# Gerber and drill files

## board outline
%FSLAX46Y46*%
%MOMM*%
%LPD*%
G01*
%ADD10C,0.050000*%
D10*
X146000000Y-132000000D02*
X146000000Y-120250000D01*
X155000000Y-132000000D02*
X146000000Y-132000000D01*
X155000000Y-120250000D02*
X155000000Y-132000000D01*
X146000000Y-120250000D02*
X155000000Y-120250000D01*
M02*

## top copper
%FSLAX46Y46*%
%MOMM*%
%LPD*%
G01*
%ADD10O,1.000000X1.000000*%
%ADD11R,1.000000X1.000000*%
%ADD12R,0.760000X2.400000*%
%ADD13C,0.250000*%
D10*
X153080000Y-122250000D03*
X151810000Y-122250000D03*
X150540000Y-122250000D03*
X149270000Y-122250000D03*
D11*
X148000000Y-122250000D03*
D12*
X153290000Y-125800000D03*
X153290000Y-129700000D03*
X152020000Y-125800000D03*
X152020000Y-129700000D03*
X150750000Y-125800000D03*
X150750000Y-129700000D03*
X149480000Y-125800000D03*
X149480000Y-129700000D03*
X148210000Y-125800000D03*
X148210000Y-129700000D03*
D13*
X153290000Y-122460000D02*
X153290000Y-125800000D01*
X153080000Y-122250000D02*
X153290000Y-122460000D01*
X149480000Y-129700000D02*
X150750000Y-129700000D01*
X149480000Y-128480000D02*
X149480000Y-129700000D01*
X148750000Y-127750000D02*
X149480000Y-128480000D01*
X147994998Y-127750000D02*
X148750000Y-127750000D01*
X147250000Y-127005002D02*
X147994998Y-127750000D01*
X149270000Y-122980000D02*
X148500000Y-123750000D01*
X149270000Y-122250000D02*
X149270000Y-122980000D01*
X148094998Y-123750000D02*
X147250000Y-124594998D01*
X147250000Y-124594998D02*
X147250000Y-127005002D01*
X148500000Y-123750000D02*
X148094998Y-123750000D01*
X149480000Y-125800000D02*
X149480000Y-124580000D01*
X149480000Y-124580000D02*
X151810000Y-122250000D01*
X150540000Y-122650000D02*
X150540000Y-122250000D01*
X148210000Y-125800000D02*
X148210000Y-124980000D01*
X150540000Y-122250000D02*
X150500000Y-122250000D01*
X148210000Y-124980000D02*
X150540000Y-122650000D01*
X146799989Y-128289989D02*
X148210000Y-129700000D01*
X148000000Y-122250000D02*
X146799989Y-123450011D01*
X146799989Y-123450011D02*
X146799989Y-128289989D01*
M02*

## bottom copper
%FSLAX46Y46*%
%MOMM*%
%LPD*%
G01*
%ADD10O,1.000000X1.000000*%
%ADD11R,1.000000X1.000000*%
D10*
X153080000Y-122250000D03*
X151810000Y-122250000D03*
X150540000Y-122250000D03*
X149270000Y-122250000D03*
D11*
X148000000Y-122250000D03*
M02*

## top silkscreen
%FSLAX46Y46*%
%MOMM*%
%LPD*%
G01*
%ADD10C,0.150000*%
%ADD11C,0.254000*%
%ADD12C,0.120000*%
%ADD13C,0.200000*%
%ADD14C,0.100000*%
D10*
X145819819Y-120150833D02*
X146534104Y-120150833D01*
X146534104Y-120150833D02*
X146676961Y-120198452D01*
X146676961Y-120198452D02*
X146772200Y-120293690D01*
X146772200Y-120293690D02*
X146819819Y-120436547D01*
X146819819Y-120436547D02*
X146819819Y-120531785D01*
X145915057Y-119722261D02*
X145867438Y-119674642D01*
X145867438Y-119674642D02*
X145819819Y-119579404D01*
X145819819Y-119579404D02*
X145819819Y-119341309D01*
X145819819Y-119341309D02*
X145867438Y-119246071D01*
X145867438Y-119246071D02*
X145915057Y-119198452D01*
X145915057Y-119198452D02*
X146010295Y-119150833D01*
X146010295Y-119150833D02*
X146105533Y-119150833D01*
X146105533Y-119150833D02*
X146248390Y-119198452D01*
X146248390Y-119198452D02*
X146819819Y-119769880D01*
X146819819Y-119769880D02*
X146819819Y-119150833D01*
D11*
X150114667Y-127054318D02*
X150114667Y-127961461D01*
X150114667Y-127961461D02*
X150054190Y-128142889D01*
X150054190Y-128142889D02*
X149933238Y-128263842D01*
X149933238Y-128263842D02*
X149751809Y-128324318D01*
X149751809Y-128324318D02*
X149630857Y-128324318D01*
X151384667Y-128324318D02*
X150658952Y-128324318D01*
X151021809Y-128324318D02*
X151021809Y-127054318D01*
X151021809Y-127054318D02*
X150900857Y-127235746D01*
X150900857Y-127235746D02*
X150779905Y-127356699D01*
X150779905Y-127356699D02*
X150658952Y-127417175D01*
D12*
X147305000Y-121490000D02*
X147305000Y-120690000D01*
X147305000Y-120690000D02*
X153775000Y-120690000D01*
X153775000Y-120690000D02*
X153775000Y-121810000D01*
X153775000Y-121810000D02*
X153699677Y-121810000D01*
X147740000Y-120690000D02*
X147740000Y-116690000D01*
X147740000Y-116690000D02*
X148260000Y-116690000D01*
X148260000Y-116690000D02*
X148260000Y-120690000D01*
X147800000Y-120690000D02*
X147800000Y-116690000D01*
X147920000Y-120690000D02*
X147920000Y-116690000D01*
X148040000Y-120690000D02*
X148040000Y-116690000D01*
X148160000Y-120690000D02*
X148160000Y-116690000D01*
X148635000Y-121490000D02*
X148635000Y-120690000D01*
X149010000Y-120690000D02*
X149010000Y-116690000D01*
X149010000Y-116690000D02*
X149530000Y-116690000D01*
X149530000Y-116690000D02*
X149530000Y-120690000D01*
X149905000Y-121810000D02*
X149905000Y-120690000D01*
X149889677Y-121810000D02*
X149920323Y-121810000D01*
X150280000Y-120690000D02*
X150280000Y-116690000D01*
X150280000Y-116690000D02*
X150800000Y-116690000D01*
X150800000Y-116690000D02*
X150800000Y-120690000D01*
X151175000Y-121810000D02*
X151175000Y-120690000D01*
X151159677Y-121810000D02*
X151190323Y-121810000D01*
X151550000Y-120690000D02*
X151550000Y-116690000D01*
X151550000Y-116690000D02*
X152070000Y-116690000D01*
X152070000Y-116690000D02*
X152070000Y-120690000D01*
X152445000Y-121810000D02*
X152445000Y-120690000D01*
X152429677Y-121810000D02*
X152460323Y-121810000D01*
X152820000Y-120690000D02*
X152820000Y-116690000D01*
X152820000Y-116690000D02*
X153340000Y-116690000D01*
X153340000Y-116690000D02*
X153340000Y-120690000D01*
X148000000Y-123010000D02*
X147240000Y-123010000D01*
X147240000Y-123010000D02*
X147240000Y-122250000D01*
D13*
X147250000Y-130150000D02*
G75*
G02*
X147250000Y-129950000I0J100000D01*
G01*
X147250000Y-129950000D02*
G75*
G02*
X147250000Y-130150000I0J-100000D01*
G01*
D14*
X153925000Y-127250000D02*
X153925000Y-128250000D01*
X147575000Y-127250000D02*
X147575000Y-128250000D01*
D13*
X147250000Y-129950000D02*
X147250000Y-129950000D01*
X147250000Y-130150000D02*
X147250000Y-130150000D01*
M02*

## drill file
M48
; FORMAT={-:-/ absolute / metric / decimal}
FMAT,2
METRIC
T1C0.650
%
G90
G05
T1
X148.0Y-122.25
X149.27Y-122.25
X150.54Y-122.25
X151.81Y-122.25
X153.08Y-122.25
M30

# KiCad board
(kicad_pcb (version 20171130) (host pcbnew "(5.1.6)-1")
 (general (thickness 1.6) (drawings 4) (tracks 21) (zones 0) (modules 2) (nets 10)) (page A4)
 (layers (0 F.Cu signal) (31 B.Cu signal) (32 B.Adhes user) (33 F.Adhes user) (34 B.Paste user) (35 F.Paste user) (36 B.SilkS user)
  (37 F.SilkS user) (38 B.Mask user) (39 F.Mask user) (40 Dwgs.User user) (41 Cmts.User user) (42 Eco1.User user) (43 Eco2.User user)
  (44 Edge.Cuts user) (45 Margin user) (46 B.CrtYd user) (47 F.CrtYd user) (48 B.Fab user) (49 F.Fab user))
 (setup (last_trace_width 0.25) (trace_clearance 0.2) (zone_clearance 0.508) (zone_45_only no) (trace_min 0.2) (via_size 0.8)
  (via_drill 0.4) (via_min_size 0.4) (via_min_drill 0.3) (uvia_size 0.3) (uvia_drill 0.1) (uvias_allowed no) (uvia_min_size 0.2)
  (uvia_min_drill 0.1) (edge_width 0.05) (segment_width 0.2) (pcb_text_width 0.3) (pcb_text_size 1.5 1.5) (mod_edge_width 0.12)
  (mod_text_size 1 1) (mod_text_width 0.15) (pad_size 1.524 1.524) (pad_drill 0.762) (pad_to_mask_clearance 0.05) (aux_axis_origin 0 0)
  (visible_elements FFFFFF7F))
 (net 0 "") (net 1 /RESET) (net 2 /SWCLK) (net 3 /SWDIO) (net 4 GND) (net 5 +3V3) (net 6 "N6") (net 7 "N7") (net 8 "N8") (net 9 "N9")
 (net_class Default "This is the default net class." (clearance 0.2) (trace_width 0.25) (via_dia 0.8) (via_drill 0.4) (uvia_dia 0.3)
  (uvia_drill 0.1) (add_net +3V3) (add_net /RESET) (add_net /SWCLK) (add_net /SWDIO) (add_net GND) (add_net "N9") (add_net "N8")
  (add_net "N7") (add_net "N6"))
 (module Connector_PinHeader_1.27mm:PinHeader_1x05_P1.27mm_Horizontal (layer F.Cu) (at 148 122.25 90)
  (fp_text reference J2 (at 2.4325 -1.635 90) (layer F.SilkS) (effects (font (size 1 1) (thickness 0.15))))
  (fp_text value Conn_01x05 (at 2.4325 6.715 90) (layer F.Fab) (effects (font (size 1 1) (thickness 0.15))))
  (fp_line (start 0.76 -0.695) (end 1.56 -0.695) (layer F.SilkS) (width 0.12))
  (fp_line (start 1.56 -0.695) (end 1.56 5.775) (layer F.SilkS) (width 0.12))
  (fp_line (start 1.56 5.775) (end 0.44 5.775) (layer F.SilkS) (width 0.12))
  (fp_line (start 0.44 5.775) (end 0.44 5.699677) (layer F.SilkS) (width 0.12))
  (fp_line (start 1.56 -0.26) (end 5.56 -0.26) (layer F.SilkS) (width 0.12))
  (fp_line (start 5.56 -0.26) (end 5.56 0.26) (layer F.SilkS) (width 0.12))
  (fp_line (start 5.56 0.26) (end 1.56 0.26) (layer F.SilkS) (width 0.12))
  (fp_line (start 1.56 -0.2) (end 5.56 -0.2) (layer F.SilkS) (width 0.12))
  (fp_line (start 1.56 -0.08) (end 5.56 -0.08) (layer F.SilkS) (width 0.12))
  (fp_line (start 1.56 0.04) (end 5.56 0.04) (layer F.SilkS) (width 0.12))
  (fp_line (start 1.56 0.16) (end 5.56 0.16) (layer F.SilkS) (width 0.12))
  (fp_line (start 0.76 0.635) (end 1.56 0.635) (layer F.SilkS) (width 0.12))
  (fp_line (start 1.56 1.01) (end 5.56 1.01) (layer F.SilkS) (width 0.12))
  (fp_line (start 5.56 1.01) (end 5.56 1.53) (layer F.SilkS) (width 0.12))
  (fp_line (start 5.56 1.53) (end 1.56 1.53) (layer F.SilkS) (width 0.12))
  (fp_line (start 0.44 1.905) (end 1.56 1.905) (layer F.SilkS) (width 0.12))
  (fp_line (start 0.44 1.889677) (end 0.44 1.920323) (layer F.SilkS) (width 0.12))
  (fp_line (start 1.56 2.28) (end 5.56 2.28) (layer F.SilkS) (width 0.12))
  (fp_line (start 5.56 2.28) (end 5.56 2.8) (layer F.SilkS) (width 0.12))
  (fp_line (start 5.56 2.8) (end 1.56 2.8) (layer F.SilkS) (width 0.12))
  (fp_line (start 0.44 3.175) (end 1.56 3.175) (layer F.SilkS) (width 0.12))
  (fp_line (start 0.44 3.159677) (end 0.44 3.190323) (layer F.SilkS) (width 0.12))
  (fp_line (start 1.56 3.55) (end 5.56 3.55) (layer F.SilkS) (width 0.12))
  (fp_line (start 5.56 3.55) (end 5.56 4.07) (layer F.SilkS) (width 0.12))
  (fp_line (start 5.56 4.07) (end 1.56 4.07) (layer F.SilkS) (width 0.12))
  (fp_line (start 0.44 4.445) (end 1.56 4.445) (layer F.SilkS) (width 0.12))
  (fp_line (start 0.44 4.429677) (end 0.44 4.460323) (layer F.SilkS) (width 0.12))
  (fp_line (start 1.56 4.82) (end 5.56 4.82) (layer F.SilkS) (width 0.12))
  (fp_line (start 5.56 4.82) (end 5.56 5.34) (layer F.SilkS) (width 0.12))
  (fp_line (start 5.56 5.34) (end 1.56 5.34) (layer F.SilkS) (width 0.12))
  (fp_line (start -0.76 0) (end -0.76 -0.76) (layer F.SilkS) (width 0.12))
  (fp_line (start -0.76 -0.76) (end 0 -0.76) (layer F.SilkS) (width 0.12))
  (pad 5 thru_hole oval (at 0 5.08 90) (size 1 1) (drill 0.65) (layers *.Cu *.Mask) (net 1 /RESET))
  (pad 4 thru_hole oval (at 0 3.81 90) (size 1 1) (drill 0.65) (layers *.Cu *.Mask) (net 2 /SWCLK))
  (pad 3 thru_hole oval (at 0 2.54 90) (size 1 1) (drill 0.65) (layers *.Cu *.Mask) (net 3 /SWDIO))
  (pad 2 thru_hole oval (at 0 1.27 90) (size 1 1) (drill 0.65) (layers *.Cu *.Mask) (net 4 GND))
  (pad 1 thru_hole rect (at 0 0 90) (size 1 1) (drill 0.65) (layers *.Cu *.Mask) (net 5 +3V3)))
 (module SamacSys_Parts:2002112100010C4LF (layer F.Cu) (at 150.75 127.75)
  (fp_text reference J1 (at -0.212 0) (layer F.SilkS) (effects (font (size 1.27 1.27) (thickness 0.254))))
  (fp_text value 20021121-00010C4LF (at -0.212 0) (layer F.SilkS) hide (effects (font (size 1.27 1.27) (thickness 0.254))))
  (fp_arc (start -3.5 2.3) (end -3.5 2.4) (angle 180) (layer F.SilkS) (width 0.2))
  (fp_arc (start -3.5 2.3) (end -3.5 2.2) (angle 180) (layer F.SilkS) (width 0.2))
  (fp_line (start 3.175 -0.5) (end 3.175 0.5) (layer F.SilkS) (width 0.1))
  (fp_line (start -3.175 -0.5) (end -3.175 0.5) (layer F.SilkS) (width 0.1))
  (fp_line (start -3.5 2.2) (end -3.5 2.2) (layer F.SilkS) (width 0.2))
  (fp_line (start -3.5 2.4) (end -3.5 2.4) (layer F.SilkS) (width 0.2))
  (pad 10 smd rect (at 2.54 -1.95) (size 0.76 2.4) (layers F.Cu F.Paste F.Mask) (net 1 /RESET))
  (pad 9 smd rect (at 2.54 1.95) (size 0.76 2.4) (layers F.Cu F.Paste F.Mask) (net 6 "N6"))
  (pad 8 smd rect (at 1.27 -1.95) (size 0.76 2.4) (layers F.Cu F.Paste F.Mask) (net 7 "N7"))
  (pad 7 smd rect (at 1.27 1.95) (size 0.76 2.4) (layers F.Cu F.Paste F.Mask) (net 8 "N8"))
  (pad 6 smd rect (at 0 -1.95) (size 0.76 2.4) (layers F.Cu F.Paste F.Mask) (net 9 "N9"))
  (pad 5 smd rect (at 0 1.95) (size 0.76 2.4) (layers F.Cu F.Paste F.Mask) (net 4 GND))
  (pad 4 smd rect (at -1.27 -1.95) (size 0.76 2.4) (layers F.Cu F.Paste F.Mask) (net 2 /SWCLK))
  (pad 3 smd rect (at -1.27 1.95) (size 0.76 2.4) (layers F.Cu F.Paste F.Mask) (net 4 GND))
  (pad 2 smd rect (at -2.54 -1.95) (size 0.76 2.4) (layers F.Cu F.Paste F.Mask) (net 3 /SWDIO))
  (pad 1 smd rect (at -2.54 1.95) (size 0.76 2.4) (layers F.Cu F.Paste F.Mask) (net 5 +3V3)))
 (gr_line (start 146 132) (end 146 120.25) (layer Edge.Cuts) (width 0.05))
 (gr_line (start 155 132) (end 146 132) (layer Edge.Cuts) (width 0.05))
 (gr_line (start 155 120.25) (end 155 132) (layer Edge.Cuts) (width 0.05))
 (gr_line (start 146 120.25) (end 155 120.25) (layer Edge.Cuts) (width 0.05))
 (segment (start 153.29 122.46) (end 153.29 125.8) (width 0.25) (layer F.Cu) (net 1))
 (segment (start 153.08 122.25) (end 153.29 122.46) (width 0.25) (layer F.Cu) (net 1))
 (segment (start 149.48 129.7) (end 150.75 129.7) (width 0.25) (layer F.Cu) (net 4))
 (segment (start 149.48 128.48) (end 149.48 129.7) (width 0.25) (layer F.Cu) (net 4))
 (segment (start 148.75 127.75) (end 149.48 128.48) (width 0.25) (layer F.Cu) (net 4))
 (segment (start 147.994998 127.75) (end 148.75 127.75) (width 0.25) (layer F.Cu) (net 4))
 (segment (start 147.25 127.005002) (end 147.994998 127.75) (width 0.25) (layer F.Cu) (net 4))
 (segment (start 149.27 122.98) (end 148.5 123.75) (width 0.25) (layer F.Cu) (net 4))
 (segment (start 149.27 122.25) (end 149.27 122.98) (width 0.25) (layer F.Cu) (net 4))
 (segment (start 148.094998 123.75) (end 147.25 124.594998) (width 0.25) (layer F.Cu) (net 4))
 (segment (start 147.25 124.594998) (end 147.25 127.005002) (width 0.25) (layer F.Cu) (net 4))
 (segment (start 148.5 123.75) (end 148.094998 123.75) (width 0.25) (layer F.Cu) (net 4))
 (segment (start 149.48 125.8) (end 149.48 124.58) (width 0.25) (layer F.Cu) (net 2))
 (segment (start 149.48 124.58) (end 151.81 122.25) (width 0.25) (layer F.Cu) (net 2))
 (segment (start 150.54 122.65) (end 150.54 122.25) (width 0.25) (layer F.Cu) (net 3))
 (segment (start 148.21 125.8) (end 148.21 124.98) (width 0.25) (layer F.Cu) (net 3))
 (segment (start 150.54 122.25) (end 150.5 122.25) (width 0.25) (layer F.Cu) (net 3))
 (segment (start 148.21 124.98) (end 150.54 122.65) (width 0.25) (layer F.Cu) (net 3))
 (segment (start 146.799989 128.289989) (end 148.21 129.7) (width 0.25) (layer F.Cu) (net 5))
 (segment (start 148 122.25) (end 146.799989 123.450011) (width 0.25) (layer F.Cu) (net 5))
 (segment (start 146.799989 123.450011) (end 146.799989 128.289989) (width 0.25) (layer F.Cu) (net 5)))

